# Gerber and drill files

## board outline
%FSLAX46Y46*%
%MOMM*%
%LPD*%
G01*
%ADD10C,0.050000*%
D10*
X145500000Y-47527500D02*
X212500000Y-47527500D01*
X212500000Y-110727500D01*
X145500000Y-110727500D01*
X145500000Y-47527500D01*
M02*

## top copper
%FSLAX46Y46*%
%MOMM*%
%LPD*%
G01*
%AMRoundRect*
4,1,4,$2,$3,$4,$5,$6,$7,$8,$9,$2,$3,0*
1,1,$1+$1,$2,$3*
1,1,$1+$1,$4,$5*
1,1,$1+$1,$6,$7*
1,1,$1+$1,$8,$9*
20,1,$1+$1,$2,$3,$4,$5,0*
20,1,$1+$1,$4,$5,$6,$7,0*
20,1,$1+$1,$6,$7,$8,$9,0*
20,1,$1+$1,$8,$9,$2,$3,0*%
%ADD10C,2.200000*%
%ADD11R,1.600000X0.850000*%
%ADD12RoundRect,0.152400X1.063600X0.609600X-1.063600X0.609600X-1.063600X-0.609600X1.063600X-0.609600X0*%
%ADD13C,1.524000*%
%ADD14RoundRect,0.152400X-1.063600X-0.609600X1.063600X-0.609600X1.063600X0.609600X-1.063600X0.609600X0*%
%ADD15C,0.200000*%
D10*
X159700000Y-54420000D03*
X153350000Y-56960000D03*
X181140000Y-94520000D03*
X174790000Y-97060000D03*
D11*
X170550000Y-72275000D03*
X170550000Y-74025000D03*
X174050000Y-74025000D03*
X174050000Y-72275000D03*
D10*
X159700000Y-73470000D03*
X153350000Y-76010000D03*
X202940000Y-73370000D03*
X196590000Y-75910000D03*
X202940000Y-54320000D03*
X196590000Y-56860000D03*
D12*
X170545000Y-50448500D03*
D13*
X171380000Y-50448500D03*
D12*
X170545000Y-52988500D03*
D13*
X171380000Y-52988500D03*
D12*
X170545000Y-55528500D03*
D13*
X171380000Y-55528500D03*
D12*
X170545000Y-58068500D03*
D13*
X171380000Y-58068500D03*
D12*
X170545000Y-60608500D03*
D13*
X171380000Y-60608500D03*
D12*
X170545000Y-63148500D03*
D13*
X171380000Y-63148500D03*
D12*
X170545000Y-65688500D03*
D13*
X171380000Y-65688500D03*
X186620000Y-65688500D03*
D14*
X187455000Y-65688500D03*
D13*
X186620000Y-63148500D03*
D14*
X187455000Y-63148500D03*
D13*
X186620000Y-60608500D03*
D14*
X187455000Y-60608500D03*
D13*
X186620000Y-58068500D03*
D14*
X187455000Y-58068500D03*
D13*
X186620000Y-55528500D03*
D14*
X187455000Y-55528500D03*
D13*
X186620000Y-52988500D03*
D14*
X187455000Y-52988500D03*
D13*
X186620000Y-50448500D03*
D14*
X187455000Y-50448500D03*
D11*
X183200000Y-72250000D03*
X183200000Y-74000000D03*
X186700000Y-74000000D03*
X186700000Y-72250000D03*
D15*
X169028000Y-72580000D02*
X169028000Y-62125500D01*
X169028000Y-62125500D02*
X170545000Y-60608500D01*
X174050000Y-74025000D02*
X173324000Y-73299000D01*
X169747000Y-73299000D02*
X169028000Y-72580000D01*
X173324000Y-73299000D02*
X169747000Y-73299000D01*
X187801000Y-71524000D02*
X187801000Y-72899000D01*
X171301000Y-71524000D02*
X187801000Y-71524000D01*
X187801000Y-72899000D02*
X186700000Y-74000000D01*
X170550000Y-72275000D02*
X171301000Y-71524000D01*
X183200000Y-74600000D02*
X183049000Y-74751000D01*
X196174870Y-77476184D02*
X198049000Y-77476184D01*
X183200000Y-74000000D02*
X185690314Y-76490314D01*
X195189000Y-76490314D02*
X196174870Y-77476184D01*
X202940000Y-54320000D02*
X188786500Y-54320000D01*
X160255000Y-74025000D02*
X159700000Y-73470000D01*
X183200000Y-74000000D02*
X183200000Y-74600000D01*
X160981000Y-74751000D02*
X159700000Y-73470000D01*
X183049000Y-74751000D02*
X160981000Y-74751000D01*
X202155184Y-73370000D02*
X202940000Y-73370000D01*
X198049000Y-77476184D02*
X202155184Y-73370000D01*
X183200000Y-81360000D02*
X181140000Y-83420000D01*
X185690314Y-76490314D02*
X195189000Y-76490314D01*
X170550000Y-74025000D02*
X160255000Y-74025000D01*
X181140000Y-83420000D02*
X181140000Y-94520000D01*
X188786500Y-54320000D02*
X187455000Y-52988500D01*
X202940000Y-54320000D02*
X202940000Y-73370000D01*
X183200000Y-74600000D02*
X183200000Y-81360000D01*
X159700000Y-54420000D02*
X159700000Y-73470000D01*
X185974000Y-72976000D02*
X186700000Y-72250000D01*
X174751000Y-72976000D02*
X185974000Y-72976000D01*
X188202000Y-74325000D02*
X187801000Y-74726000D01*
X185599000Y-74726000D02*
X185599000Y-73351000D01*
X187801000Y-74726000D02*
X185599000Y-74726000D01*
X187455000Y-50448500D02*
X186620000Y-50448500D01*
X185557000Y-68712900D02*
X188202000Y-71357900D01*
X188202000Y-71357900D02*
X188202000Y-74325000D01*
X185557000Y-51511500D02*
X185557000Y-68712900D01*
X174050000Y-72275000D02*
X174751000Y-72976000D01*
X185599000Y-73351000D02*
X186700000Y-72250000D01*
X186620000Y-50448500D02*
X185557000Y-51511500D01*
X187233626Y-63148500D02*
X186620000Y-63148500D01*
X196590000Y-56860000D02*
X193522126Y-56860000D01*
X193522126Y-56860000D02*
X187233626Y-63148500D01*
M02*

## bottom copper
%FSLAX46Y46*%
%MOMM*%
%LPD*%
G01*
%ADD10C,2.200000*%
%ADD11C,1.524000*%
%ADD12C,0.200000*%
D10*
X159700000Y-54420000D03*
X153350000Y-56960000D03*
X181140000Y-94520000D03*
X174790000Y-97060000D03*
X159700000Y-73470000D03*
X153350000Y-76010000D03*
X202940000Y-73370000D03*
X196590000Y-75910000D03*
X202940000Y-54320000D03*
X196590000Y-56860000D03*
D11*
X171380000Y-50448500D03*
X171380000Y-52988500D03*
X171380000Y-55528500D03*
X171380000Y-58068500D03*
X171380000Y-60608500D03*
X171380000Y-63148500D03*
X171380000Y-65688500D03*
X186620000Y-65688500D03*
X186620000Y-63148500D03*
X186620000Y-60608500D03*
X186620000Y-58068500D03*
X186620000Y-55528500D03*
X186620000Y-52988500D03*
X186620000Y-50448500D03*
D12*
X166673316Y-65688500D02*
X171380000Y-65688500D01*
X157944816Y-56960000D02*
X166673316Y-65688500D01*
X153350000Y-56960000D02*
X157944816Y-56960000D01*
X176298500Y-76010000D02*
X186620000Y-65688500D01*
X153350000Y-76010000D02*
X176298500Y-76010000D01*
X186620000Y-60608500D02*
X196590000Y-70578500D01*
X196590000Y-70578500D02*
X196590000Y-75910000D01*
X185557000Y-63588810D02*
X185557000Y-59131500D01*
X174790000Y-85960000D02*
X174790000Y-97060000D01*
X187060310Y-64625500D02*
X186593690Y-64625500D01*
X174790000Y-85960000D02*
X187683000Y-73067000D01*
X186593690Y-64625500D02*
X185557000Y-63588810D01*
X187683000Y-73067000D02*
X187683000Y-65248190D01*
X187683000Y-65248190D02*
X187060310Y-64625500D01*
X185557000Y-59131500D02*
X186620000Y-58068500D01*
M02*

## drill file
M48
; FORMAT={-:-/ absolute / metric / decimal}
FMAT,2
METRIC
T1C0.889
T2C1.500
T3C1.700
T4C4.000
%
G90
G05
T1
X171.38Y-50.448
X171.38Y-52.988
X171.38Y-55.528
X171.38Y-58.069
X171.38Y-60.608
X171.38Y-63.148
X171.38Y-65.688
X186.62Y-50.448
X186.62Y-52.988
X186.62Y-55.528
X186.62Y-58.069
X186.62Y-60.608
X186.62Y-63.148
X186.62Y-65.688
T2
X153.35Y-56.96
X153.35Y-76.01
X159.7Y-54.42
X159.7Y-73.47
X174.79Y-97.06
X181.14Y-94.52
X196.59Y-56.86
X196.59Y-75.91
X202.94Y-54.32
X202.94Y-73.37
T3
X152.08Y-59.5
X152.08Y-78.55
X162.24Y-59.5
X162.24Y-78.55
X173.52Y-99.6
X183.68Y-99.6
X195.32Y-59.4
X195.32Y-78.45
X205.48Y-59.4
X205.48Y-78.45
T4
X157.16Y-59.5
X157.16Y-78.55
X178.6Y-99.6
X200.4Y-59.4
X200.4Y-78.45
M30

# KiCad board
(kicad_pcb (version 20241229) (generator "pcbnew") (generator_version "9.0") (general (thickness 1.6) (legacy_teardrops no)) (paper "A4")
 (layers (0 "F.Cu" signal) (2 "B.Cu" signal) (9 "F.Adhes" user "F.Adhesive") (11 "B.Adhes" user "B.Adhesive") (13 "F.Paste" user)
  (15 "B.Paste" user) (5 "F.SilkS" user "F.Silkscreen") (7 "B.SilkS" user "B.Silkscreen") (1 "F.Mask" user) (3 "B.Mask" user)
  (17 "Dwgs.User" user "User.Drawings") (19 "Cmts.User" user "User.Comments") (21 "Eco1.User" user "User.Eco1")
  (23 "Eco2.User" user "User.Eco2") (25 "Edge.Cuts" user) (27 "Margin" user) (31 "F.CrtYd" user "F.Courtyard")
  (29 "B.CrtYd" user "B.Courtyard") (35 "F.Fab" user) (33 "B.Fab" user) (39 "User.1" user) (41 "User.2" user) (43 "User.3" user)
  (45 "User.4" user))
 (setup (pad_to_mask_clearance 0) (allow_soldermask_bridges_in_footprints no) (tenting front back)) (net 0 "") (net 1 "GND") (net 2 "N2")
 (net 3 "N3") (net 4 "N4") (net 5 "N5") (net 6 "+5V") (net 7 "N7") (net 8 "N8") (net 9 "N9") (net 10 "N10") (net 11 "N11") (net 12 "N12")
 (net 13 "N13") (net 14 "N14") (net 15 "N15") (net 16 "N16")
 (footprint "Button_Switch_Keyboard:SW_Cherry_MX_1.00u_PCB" (layer "F.Cu") (at 159.7 54.42)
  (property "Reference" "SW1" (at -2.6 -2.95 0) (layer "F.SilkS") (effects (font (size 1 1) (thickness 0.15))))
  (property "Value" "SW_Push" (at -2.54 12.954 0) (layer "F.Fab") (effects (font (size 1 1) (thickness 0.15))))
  (pad "" np_thru_hole circle (at -7.62 5.08) (size 1.7 1.7) (drill 1.7) (layers "*.Cu" "*.Mask"))
  (pad "" np_thru_hole circle (at -2.54 5.08) (size 4 4) (drill 4) (layers "*.Cu" "*.Mask"))
  (pad "" np_thru_hole circle (at 2.54 5.08) (size 1.7 1.7) (drill 1.7) (layers "*.Cu" "*.Mask"))
  (pad "1" thru_hole circle (at 0 0) (size 2.2 2.2) (drill 1.5) (layers "*.Cu" "*.Mask") (remove_unused_layers no) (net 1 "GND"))
  (pad "2" thru_hole circle (at -6.35 2.54) (size 2.2 2.2) (drill 1.5) (layers "*.Cu" "*.Mask") (remove_unused_layers no) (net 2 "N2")))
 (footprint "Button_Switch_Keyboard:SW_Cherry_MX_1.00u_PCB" (layer "F.Cu") (at 181.14 94.52)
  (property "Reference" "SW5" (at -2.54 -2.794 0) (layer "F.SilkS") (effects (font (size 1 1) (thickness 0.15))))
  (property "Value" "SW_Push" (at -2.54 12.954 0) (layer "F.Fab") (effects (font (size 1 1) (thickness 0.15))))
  (pad "" np_thru_hole circle (at -7.62 5.08) (size 1.7 1.7) (drill 1.7) (layers "*.Cu" "*.Mask"))
  (pad "" np_thru_hole circle (at -2.54 5.08) (size 4 4) (drill 4) (layers "*.Cu" "*.Mask"))
  (pad "" np_thru_hole circle (at 2.54 5.08) (size 1.7 1.7) (drill 1.7) (layers "*.Cu" "*.Mask"))
  (pad "1" thru_hole circle (at 0 0) (size 2.2 2.2) (drill 1.5) (layers "*.Cu" "*.Mask") (remove_unused_layers no) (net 1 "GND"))
  (pad "2" thru_hole circle (at -6.35 2.54) (size 2.2 2.2) (drill 1.5) (layers "*.Cu" "*.Mask") (remove_unused_layers no) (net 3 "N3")))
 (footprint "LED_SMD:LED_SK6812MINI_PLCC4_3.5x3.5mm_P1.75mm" (layer "F.Cu") (at 172.3 73.15)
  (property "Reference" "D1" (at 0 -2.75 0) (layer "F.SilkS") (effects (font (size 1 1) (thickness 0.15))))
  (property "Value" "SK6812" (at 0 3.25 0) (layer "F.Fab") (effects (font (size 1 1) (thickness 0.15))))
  (pad "1" smd rect (at -1.75 -0.875) (size 1.6 0.85) (layers "F.Cu" "F.Mask" "F.Paste") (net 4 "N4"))
  (pad "2" smd rect (at -1.75 0.875) (size 1.6 0.85) (layers "F.Cu" "F.Mask" "F.Paste") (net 1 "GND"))
  (pad "3" smd rect (at 1.75 0.875) (size 1.6 0.85) (layers "F.Cu" "F.Mask" "F.Paste") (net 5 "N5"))
  (pad "4" smd rect (at 1.75 -0.875) (size 1.6 0.85) (layers "F.Cu" "F.Mask" "F.Paste") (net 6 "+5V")))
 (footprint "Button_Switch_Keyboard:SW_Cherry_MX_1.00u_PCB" (layer "F.Cu") (at 159.7 73.47)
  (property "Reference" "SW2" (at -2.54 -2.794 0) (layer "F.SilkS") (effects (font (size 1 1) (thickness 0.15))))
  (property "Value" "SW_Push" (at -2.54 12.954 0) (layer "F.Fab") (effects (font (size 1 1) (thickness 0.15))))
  (pad "" np_thru_hole circle (at -7.62 5.08) (size 1.7 1.7) (drill 1.7) (layers "*.Cu" "*.Mask"))
  (pad "" np_thru_hole circle (at -2.54 5.08) (size 4 4) (drill 4) (layers "*.Cu" "*.Mask"))
  (pad "" np_thru_hole circle (at 2.54 5.08) (size 1.7 1.7) (drill 1.7) (layers "*.Cu" "*.Mask"))
  (pad "1" thru_hole circle (at 0 0) (size 2.2 2.2) (drill 1.5) (layers "*.Cu" "*.Mask") (remove_unused_layers no) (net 1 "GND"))
  (pad "2" thru_hole circle (at -6.35 2.54) (size 2.2 2.2) (drill 1.5) (layers "*.Cu" "*.Mask") (remove_unused_layers no) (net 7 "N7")))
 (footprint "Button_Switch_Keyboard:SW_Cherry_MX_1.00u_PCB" (layer "F.Cu") (at 202.94 73.37)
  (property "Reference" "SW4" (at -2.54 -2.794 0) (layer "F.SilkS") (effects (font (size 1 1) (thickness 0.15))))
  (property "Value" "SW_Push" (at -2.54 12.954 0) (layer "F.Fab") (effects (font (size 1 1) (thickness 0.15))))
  (pad "" np_thru_hole circle (at -7.62 5.08) (size 1.7 1.7) (drill 1.7) (layers "*.Cu" "*.Mask"))
  (pad "" np_thru_hole circle (at -2.54 5.08) (size 4 4) (drill 4) (layers "*.Cu" "*.Mask"))
  (pad "" np_thru_hole circle (at 2.54 5.08) (size 1.7 1.7) (drill 1.7) (layers "*.Cu" "*.Mask"))
  (pad "1" thru_hole circle (at 0 0) (size 2.2 2.2) (drill 1.5) (layers "*.Cu" "*.Mask") (remove_unused_layers no) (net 1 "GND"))
  (pad "2" thru_hole circle (at -6.35 2.54) (size 2.2 2.2) (drill 1.5) (layers "*.Cu" "*.Mask") (remove_unused_layers no) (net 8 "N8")))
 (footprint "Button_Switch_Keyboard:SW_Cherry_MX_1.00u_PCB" (layer "F.Cu") (at 202.94 54.32)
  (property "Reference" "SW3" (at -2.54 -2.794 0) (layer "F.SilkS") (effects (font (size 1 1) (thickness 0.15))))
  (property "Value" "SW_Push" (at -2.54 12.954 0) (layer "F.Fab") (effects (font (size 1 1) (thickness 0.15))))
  (pad "" np_thru_hole circle (at -7.62 5.08) (size 1.7 1.7) (drill 1.7) (layers "*.Cu" "*.Mask"))
  (pad "" np_thru_hole circle (at -2.54 5.08) (size 4 4) (drill 4) (layers "*.Cu" "*.Mask"))
  (pad "" np_thru_hole circle (at 2.54 5.08) (size 1.7 1.7) (drill 1.7) (layers "*.Cu" "*.Mask"))
  (pad "1" thru_hole circle (at 0 0) (size 2.2 2.2) (drill 1.5) (layers "*.Cu" "*.Mask") (remove_unused_layers no) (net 1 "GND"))
  (pad "2" thru_hole circle (at -6.35 2.54) (size 2.2 2.2) (drill 1.5) (layers "*.Cu" "*.Mask") (remove_unused_layers no) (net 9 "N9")))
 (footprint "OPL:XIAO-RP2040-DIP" (layer "F.Cu") (at 179 58.0685)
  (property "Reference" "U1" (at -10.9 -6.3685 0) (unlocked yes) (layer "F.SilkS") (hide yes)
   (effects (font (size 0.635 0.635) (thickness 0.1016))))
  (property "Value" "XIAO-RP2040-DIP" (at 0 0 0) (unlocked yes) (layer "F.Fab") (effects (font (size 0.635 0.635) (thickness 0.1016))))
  (pad "1" smd roundrect (at -8.455 -7.62 180) (size 2.432 1.524) (layers "F.Cu" "F.Mask") (roundrect_rratio 0.1) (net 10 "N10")
   (thermal_bridge_angle 45))
  (pad "1" thru_hole circle (at -7.62 -7.62 180) (size 1.524 1.524) (drill 0.889) (layers "*.Cu" "*.Mask") (remove_unused_layers no)
   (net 10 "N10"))
  (pad "2" smd roundrect (at -8.455 -5.08 180) (size 2.432 1.524) (layers "F.Cu" "F.Mask") (roundrect_rratio 0.1) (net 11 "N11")
   (thermal_bridge_angle 45))
  (pad "2" thru_hole circle (at -7.62 -5.08 180) (size 1.524 1.524) (drill 0.889) (layers "*.Cu" "*.Mask") (remove_unused_layers no)
   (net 11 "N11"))
  (pad "3" smd roundrect (at -8.455 -2.54 180) (size 2.432 1.524) (layers "F.Cu" "F.Mask") (roundrect_rratio 0.1) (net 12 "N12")
   (thermal_bridge_angle 45))
  (pad "3" thru_hole circle (at -7.62 -2.54 180) (size 1.524 1.524) (drill 0.889) (layers "*.Cu" "*.Mask") (remove_unused_layers no)
   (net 12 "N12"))
  (pad "4" smd roundrect (at -8.455 0 180) (size 2.432 1.524) (layers "F.Cu" "F.Mask") (roundrect_rratio 0.1) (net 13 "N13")
   (thermal_bridge_angle 45))
  (pad "4" thru_hole circle (at -7.62 0 180) (size 1.524 1.524) (drill 0.889) (layers "*.Cu" "*.Mask") (remove_unused_layers no)
   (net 13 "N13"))
  (pad "5" smd roundrect (at -8.455 2.54 180) (size 2.432 1.524) (layers "F.Cu" "F.Mask") (roundrect_rratio 0.1) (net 5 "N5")
   (thermal_bridge_angle 45))
  (pad "5" thru_hole circle (at -7.62 2.54 180) (size 1.524 1.524) (drill 0.889) (layers "*.Cu" "*.Mask") (remove_unused_layers no)
   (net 5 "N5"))
  (pad "6" smd roundrect (at -8.455 5.08 180) (size 2.432 1.524) (layers "F.Cu" "F.Mask") (roundrect_rratio 0.1) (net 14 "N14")
   (thermal_bridge_angle 45))
  (pad "6" thru_hole circle (at -7.62 5.08 180) (size 1.524 1.524) (drill 0.889) (layers "*.Cu" "*.Mask") (remove_unused_layers no)
   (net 14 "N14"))
  (pad "7" smd roundrect (at -8.455 7.62 180) (size 2.432 1.524) (layers "F.Cu" "F.Mask") (roundrect_rratio 0.1) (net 2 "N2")
   (thermal_bridge_angle 45))
  (pad "7" thru_hole circle (at -7.62 7.62 180) (size 1.524 1.524) (drill 0.889) (layers "*.Cu" "*.Mask") (remove_unused_layers no)
   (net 2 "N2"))
  (pad "8" thru_hole circle (at 7.62 7.62) (size 1.524 1.524) (drill 0.889) (layers "*.Cu" "*.Mask") (remove_unused_layers no) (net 7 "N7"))
  (pad "8" smd roundrect (at 8.455 7.62) (size 2.432 1.524) (layers "F.Cu" "F.Mask") (roundrect_rratio 0.1) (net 7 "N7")
   (thermal_bridge_angle 45))
  (pad "9" thru_hole circle (at 7.62 5.08) (size 1.524 1.524) (drill 0.889) (layers "*.Cu" "*.Mask") (remove_unused_layers no) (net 9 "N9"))
  (pad "9" smd roundrect (at 8.455 5.08) (size 2.432 1.524) (layers "F.Cu" "F.Mask") (roundrect_rratio 0.1) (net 9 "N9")
   (thermal_bridge_angle 45))
  (pad "10" thru_hole circle (at 7.62 2.54) (size 1.524 1.524) (drill 0.889) (layers "*.Cu" "*.Mask") (remove_unused_layers no) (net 8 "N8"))
  (pad "10" smd roundrect (at 8.455 2.54) (size 2.432 1.524) (layers "F.Cu" "F.Mask") (roundrect_rratio 0.1) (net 8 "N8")
   (thermal_bridge_angle 45))
  (pad "11" thru_hole circle (at 7.62 0) (size 1.524 1.524) (drill 0.889) (layers "*.Cu" "*.Mask") (remove_unused_layers no) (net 3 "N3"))
  (pad "11" smd roundrect (at 8.455 0) (size 2.432 1.524) (layers "F.Cu" "F.Mask") (roundrect_rratio 0.1) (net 3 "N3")
   (thermal_bridge_angle 45))
  (pad "12" thru_hole circle (at 7.62 -2.54) (size 1.524 1.524) (drill 0.889) (layers "*.Cu" "*.Mask") (remove_unused_layers no)
   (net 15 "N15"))
  (pad "12" smd roundrect (at 8.455 -2.54) (size 2.432 1.524) (layers "F.Cu" "F.Mask") (roundrect_rratio 0.1) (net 15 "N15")
   (thermal_bridge_angle 45))
  (pad "13" thru_hole circle (at 7.62 -5.08) (size 1.524 1.524) (drill 0.889) (layers "*.Cu" "*.Mask") (remove_unused_layers no)
   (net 1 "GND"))
  (pad "13" smd roundrect (at 8.455 -5.08) (size 2.432 1.524) (layers "F.Cu" "F.Mask") (roundrect_rratio 0.1) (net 1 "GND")
   (thermal_bridge_angle 45))
  (pad "14" thru_hole circle (at 7.62 -7.62) (size 1.524 1.524) (drill 0.889) (layers "*.Cu" "*.Mask") (remove_unused_layers no)
   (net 6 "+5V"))
  (pad "14" smd roundrect (at 8.455 -7.62) (size 2.432 1.524) (layers "F.Cu" "F.Mask") (roundrect_rratio 0.1) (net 6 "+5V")
   (thermal_bridge_angle 45)))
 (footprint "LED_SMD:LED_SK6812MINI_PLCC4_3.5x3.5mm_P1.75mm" (layer "F.Cu") (at 184.95 73.125)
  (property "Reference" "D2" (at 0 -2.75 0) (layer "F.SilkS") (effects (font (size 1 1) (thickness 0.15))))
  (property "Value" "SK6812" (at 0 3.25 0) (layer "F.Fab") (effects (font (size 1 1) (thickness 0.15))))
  (pad "1" smd rect (at -1.75 -0.875) (size 1.6 0.85) (layers "F.Cu" "F.Mask" "F.Paste") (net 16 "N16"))
  (pad "2" smd rect (at -1.75 0.875) (size 1.6 0.85) (layers "F.Cu" "F.Mask" "F.Paste") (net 1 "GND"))
  (pad "3" smd rect (at 1.75 0.875) (size 1.6 0.85) (layers "F.Cu" "F.Mask" "F.Paste") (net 4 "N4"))
  (pad "4" smd rect (at 1.75 -0.875) (size 1.6 0.85) (layers "F.Cu" "F.Mask" "F.Paste") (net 6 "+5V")))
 (gr_rect (start 145.5 47.5275) (end 212.5 110.7275) (stroke (width 0.05) (type default)) (fill no) (layer "Edge.Cuts"))
 (segment (start 169.028 72.58) (end 169.028 62.1255) (width 0.2) (layer "F.Cu") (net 5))
 (segment (start 169.028 62.1255) (end 170.545 60.6085) (width 0.2) (layer "F.Cu") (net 5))
 (segment (start 174.05 74.025) (end 173.324 73.299) (width 0.2) (layer "F.Cu") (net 5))
 (segment (start 169.747 73.299) (end 169.028 72.58) (width 0.2) (layer "F.Cu") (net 5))
 (segment (start 173.324 73.299) (end 169.747 73.299) (width 0.2) (layer "F.Cu") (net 5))
 (segment (start 187.801 71.524) (end 187.801 72.899) (width 0.2) (layer "F.Cu") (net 4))
 (segment (start 171.301 71.524) (end 187.801 71.524) (width 0.2) (layer "F.Cu") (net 4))
 (segment (start 187.801 72.899) (end 186.7 74) (width 0.2) (layer "F.Cu") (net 4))
 (segment (start 170.55 72.275) (end 171.301 71.524) (width 0.2) (layer "F.Cu") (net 4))
 (segment (start 183.2 74.6) (end 183.049 74.751) (width 0.2) (layer "F.Cu") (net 1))
 (segment (start 196.17487 77.476184) (end 198.049 77.476184) (width 0.2) (layer "F.Cu") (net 1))
 (segment (start 183.2 74) (end 185.690314 76.490314) (width 0.2) (layer "F.Cu") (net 1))
 (segment (start 195.189 76.490314) (end 196.17487 77.476184) (width 0.2) (layer "F.Cu") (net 1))
 (segment (start 202.94 54.32) (end 188.7865 54.32) (width 0.2) (layer "F.Cu") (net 1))
 (segment (start 160.255 74.025) (end 159.7 73.47) (width 0.2) (layer "F.Cu") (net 1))
 (segment (start 183.2 74) (end 183.2 74.6) (width 0.2) (layer "F.Cu") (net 1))
 (segment (start 160.981 74.751) (end 159.7 73.47) (width 0.2) (layer "F.Cu") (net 1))
 (segment (start 183.049 74.751) (end 160.981 74.751) (width 0.2) (layer "F.Cu") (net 1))
 (segment (start 202.155184 73.37) (end 202.94 73.37) (width 0.2) (layer "F.Cu") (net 1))
 (segment (start 198.049 77.476184) (end 202.155184 73.37) (width 0.2) (layer "F.Cu") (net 1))
 (segment (start 183.2 81.36) (end 181.14 83.42) (width 0.2) (layer "F.Cu") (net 1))
 (segment (start 185.690314 76.490314) (end 195.189 76.490314) (width 0.2) (layer "F.Cu") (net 1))
 (segment (start 170.55 74.025) (end 160.255 74.025) (width 0.2) (layer "F.Cu") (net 1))
 (segment (start 181.14 83.42) (end 181.14 94.52) (width 0.2) (layer "F.Cu") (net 1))
 (segment (start 188.7865 54.32) (end 187.455 52.9885) (width 0.2) (layer "F.Cu") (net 1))
 (segment (start 202.94 54.32) (end 202.94 73.37) (width 0.2) (layer "F.Cu") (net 1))
 (segment (start 183.2 74.6) (end 183.2 81.36) (width 0.2) (layer "F.Cu") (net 1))
 (segment (start 159.7 54.42) (end 159.7 73.47) (width 0.2) (layer "F.Cu") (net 1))
 (segment (start 185.974 72.976) (end 186.7 72.25) (width 0.2) (layer "F.Cu") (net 6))
 (segment (start 174.751 72.976) (end 185.974 72.976) (width 0.2) (layer "F.Cu") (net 6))
 (segment (start 188.202 74.325) (end 187.801 74.726) (width 0.2) (layer "F.Cu") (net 6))
 (segment (start 185.599 74.726) (end 185.599 73.351) (width 0.2) (layer "F.Cu") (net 6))
 (segment (start 187.801 74.726) (end 185.599 74.726) (width 0.2) (layer "F.Cu") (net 6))
 (segment (start 187.455 50.4485) (end 186.62 50.4485) (width 0.2) (layer "F.Cu") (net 6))
 (segment (start 185.557 68.7129) (end 188.202 71.3579) (width 0.2) (layer "F.Cu") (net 6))
 (segment (start 188.202 71.3579) (end 188.202 74.325) (width 0.2) (layer "F.Cu") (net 6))
 (segment (start 185.557 51.5115) (end 185.557 68.7129) (width 0.2) (layer "F.Cu") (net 6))
 (segment (start 174.05 72.275) (end 174.751 72.976) (width 0.2) (layer "F.Cu") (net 6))
 (segment (start 185.599 73.351) (end 186.7 72.25) (width 0.2) (layer "F.Cu") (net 6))
 (segment (start 186.62 50.4485) (end 185.557 51.5115) (width 0.2) (layer "F.Cu") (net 6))
 (segment (start 166.673316 65.6885) (end 171.38 65.6885) (width 0.2) (layer "B.Cu") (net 2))
 (segment (start 157.944816 56.96) (end 166.673316 65.6885) (width 0.2) (layer "B.Cu") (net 2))
 (segment (start 153.35 56.96) (end 157.944816 56.96) (width 0.2) (layer "B.Cu") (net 2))
 (segment (start 176.2985 76.01) (end 186.62 65.6885) (width 0.2) (layer "B.Cu") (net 7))
 (segment (start 153.35 76.01) (end 176.2985 76.01) (width 0.2) (layer "B.Cu") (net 7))
 (segment (start 187.233626 63.1485) (end 186.62 63.1485) (width 0.2) (layer "F.Cu") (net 9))
 (segment (start 196.59 56.86) (end 193.522126 56.86) (width 0.2) (layer "F.Cu") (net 9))
 (segment (start 193.522126 56.86) (end 187.233626 63.1485) (width 0.2) (layer "F.Cu") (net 9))
 (segment (start 186.62 60.6085) (end 196.59 70.5785) (width 0.2) (layer "B.Cu") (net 8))
 (segment (start 196.59 70.5785) (end 196.59 75.91) (width 0.2) (layer "B.Cu") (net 8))
 (segment (start 185.557 63.58881) (end 185.557 59.1315) (width 0.2) (layer "B.Cu") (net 3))
 (segment (start 174.79 85.96) (end 174.79 97.06) (width 0.2) (layer "B.Cu") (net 3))
 (segment (start 187.06031 64.6255) (end 186.59369 64.6255) (width 0.2) (layer "B.Cu") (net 3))
 (segment (start 174.79 85.96) (end 187.683 73.067) (width 0.2) (layer "B.Cu") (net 3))
 (segment (start 186.59369 64.6255) (end 185.557 63.58881) (width 0.2) (layer "B.Cu") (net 3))
 (segment (start 187.683 73.067) (end 187.683 65.24819) (width 0.2) (layer "B.Cu") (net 3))
 (segment (start 187.683 65.24819) (end 187.06031 64.6255) (width 0.2) (layer "B.Cu") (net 3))
 (segment (start 185.557 59.1315) (end 186.62 58.0685) (width 0.2) (layer "B.Cu") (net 3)))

